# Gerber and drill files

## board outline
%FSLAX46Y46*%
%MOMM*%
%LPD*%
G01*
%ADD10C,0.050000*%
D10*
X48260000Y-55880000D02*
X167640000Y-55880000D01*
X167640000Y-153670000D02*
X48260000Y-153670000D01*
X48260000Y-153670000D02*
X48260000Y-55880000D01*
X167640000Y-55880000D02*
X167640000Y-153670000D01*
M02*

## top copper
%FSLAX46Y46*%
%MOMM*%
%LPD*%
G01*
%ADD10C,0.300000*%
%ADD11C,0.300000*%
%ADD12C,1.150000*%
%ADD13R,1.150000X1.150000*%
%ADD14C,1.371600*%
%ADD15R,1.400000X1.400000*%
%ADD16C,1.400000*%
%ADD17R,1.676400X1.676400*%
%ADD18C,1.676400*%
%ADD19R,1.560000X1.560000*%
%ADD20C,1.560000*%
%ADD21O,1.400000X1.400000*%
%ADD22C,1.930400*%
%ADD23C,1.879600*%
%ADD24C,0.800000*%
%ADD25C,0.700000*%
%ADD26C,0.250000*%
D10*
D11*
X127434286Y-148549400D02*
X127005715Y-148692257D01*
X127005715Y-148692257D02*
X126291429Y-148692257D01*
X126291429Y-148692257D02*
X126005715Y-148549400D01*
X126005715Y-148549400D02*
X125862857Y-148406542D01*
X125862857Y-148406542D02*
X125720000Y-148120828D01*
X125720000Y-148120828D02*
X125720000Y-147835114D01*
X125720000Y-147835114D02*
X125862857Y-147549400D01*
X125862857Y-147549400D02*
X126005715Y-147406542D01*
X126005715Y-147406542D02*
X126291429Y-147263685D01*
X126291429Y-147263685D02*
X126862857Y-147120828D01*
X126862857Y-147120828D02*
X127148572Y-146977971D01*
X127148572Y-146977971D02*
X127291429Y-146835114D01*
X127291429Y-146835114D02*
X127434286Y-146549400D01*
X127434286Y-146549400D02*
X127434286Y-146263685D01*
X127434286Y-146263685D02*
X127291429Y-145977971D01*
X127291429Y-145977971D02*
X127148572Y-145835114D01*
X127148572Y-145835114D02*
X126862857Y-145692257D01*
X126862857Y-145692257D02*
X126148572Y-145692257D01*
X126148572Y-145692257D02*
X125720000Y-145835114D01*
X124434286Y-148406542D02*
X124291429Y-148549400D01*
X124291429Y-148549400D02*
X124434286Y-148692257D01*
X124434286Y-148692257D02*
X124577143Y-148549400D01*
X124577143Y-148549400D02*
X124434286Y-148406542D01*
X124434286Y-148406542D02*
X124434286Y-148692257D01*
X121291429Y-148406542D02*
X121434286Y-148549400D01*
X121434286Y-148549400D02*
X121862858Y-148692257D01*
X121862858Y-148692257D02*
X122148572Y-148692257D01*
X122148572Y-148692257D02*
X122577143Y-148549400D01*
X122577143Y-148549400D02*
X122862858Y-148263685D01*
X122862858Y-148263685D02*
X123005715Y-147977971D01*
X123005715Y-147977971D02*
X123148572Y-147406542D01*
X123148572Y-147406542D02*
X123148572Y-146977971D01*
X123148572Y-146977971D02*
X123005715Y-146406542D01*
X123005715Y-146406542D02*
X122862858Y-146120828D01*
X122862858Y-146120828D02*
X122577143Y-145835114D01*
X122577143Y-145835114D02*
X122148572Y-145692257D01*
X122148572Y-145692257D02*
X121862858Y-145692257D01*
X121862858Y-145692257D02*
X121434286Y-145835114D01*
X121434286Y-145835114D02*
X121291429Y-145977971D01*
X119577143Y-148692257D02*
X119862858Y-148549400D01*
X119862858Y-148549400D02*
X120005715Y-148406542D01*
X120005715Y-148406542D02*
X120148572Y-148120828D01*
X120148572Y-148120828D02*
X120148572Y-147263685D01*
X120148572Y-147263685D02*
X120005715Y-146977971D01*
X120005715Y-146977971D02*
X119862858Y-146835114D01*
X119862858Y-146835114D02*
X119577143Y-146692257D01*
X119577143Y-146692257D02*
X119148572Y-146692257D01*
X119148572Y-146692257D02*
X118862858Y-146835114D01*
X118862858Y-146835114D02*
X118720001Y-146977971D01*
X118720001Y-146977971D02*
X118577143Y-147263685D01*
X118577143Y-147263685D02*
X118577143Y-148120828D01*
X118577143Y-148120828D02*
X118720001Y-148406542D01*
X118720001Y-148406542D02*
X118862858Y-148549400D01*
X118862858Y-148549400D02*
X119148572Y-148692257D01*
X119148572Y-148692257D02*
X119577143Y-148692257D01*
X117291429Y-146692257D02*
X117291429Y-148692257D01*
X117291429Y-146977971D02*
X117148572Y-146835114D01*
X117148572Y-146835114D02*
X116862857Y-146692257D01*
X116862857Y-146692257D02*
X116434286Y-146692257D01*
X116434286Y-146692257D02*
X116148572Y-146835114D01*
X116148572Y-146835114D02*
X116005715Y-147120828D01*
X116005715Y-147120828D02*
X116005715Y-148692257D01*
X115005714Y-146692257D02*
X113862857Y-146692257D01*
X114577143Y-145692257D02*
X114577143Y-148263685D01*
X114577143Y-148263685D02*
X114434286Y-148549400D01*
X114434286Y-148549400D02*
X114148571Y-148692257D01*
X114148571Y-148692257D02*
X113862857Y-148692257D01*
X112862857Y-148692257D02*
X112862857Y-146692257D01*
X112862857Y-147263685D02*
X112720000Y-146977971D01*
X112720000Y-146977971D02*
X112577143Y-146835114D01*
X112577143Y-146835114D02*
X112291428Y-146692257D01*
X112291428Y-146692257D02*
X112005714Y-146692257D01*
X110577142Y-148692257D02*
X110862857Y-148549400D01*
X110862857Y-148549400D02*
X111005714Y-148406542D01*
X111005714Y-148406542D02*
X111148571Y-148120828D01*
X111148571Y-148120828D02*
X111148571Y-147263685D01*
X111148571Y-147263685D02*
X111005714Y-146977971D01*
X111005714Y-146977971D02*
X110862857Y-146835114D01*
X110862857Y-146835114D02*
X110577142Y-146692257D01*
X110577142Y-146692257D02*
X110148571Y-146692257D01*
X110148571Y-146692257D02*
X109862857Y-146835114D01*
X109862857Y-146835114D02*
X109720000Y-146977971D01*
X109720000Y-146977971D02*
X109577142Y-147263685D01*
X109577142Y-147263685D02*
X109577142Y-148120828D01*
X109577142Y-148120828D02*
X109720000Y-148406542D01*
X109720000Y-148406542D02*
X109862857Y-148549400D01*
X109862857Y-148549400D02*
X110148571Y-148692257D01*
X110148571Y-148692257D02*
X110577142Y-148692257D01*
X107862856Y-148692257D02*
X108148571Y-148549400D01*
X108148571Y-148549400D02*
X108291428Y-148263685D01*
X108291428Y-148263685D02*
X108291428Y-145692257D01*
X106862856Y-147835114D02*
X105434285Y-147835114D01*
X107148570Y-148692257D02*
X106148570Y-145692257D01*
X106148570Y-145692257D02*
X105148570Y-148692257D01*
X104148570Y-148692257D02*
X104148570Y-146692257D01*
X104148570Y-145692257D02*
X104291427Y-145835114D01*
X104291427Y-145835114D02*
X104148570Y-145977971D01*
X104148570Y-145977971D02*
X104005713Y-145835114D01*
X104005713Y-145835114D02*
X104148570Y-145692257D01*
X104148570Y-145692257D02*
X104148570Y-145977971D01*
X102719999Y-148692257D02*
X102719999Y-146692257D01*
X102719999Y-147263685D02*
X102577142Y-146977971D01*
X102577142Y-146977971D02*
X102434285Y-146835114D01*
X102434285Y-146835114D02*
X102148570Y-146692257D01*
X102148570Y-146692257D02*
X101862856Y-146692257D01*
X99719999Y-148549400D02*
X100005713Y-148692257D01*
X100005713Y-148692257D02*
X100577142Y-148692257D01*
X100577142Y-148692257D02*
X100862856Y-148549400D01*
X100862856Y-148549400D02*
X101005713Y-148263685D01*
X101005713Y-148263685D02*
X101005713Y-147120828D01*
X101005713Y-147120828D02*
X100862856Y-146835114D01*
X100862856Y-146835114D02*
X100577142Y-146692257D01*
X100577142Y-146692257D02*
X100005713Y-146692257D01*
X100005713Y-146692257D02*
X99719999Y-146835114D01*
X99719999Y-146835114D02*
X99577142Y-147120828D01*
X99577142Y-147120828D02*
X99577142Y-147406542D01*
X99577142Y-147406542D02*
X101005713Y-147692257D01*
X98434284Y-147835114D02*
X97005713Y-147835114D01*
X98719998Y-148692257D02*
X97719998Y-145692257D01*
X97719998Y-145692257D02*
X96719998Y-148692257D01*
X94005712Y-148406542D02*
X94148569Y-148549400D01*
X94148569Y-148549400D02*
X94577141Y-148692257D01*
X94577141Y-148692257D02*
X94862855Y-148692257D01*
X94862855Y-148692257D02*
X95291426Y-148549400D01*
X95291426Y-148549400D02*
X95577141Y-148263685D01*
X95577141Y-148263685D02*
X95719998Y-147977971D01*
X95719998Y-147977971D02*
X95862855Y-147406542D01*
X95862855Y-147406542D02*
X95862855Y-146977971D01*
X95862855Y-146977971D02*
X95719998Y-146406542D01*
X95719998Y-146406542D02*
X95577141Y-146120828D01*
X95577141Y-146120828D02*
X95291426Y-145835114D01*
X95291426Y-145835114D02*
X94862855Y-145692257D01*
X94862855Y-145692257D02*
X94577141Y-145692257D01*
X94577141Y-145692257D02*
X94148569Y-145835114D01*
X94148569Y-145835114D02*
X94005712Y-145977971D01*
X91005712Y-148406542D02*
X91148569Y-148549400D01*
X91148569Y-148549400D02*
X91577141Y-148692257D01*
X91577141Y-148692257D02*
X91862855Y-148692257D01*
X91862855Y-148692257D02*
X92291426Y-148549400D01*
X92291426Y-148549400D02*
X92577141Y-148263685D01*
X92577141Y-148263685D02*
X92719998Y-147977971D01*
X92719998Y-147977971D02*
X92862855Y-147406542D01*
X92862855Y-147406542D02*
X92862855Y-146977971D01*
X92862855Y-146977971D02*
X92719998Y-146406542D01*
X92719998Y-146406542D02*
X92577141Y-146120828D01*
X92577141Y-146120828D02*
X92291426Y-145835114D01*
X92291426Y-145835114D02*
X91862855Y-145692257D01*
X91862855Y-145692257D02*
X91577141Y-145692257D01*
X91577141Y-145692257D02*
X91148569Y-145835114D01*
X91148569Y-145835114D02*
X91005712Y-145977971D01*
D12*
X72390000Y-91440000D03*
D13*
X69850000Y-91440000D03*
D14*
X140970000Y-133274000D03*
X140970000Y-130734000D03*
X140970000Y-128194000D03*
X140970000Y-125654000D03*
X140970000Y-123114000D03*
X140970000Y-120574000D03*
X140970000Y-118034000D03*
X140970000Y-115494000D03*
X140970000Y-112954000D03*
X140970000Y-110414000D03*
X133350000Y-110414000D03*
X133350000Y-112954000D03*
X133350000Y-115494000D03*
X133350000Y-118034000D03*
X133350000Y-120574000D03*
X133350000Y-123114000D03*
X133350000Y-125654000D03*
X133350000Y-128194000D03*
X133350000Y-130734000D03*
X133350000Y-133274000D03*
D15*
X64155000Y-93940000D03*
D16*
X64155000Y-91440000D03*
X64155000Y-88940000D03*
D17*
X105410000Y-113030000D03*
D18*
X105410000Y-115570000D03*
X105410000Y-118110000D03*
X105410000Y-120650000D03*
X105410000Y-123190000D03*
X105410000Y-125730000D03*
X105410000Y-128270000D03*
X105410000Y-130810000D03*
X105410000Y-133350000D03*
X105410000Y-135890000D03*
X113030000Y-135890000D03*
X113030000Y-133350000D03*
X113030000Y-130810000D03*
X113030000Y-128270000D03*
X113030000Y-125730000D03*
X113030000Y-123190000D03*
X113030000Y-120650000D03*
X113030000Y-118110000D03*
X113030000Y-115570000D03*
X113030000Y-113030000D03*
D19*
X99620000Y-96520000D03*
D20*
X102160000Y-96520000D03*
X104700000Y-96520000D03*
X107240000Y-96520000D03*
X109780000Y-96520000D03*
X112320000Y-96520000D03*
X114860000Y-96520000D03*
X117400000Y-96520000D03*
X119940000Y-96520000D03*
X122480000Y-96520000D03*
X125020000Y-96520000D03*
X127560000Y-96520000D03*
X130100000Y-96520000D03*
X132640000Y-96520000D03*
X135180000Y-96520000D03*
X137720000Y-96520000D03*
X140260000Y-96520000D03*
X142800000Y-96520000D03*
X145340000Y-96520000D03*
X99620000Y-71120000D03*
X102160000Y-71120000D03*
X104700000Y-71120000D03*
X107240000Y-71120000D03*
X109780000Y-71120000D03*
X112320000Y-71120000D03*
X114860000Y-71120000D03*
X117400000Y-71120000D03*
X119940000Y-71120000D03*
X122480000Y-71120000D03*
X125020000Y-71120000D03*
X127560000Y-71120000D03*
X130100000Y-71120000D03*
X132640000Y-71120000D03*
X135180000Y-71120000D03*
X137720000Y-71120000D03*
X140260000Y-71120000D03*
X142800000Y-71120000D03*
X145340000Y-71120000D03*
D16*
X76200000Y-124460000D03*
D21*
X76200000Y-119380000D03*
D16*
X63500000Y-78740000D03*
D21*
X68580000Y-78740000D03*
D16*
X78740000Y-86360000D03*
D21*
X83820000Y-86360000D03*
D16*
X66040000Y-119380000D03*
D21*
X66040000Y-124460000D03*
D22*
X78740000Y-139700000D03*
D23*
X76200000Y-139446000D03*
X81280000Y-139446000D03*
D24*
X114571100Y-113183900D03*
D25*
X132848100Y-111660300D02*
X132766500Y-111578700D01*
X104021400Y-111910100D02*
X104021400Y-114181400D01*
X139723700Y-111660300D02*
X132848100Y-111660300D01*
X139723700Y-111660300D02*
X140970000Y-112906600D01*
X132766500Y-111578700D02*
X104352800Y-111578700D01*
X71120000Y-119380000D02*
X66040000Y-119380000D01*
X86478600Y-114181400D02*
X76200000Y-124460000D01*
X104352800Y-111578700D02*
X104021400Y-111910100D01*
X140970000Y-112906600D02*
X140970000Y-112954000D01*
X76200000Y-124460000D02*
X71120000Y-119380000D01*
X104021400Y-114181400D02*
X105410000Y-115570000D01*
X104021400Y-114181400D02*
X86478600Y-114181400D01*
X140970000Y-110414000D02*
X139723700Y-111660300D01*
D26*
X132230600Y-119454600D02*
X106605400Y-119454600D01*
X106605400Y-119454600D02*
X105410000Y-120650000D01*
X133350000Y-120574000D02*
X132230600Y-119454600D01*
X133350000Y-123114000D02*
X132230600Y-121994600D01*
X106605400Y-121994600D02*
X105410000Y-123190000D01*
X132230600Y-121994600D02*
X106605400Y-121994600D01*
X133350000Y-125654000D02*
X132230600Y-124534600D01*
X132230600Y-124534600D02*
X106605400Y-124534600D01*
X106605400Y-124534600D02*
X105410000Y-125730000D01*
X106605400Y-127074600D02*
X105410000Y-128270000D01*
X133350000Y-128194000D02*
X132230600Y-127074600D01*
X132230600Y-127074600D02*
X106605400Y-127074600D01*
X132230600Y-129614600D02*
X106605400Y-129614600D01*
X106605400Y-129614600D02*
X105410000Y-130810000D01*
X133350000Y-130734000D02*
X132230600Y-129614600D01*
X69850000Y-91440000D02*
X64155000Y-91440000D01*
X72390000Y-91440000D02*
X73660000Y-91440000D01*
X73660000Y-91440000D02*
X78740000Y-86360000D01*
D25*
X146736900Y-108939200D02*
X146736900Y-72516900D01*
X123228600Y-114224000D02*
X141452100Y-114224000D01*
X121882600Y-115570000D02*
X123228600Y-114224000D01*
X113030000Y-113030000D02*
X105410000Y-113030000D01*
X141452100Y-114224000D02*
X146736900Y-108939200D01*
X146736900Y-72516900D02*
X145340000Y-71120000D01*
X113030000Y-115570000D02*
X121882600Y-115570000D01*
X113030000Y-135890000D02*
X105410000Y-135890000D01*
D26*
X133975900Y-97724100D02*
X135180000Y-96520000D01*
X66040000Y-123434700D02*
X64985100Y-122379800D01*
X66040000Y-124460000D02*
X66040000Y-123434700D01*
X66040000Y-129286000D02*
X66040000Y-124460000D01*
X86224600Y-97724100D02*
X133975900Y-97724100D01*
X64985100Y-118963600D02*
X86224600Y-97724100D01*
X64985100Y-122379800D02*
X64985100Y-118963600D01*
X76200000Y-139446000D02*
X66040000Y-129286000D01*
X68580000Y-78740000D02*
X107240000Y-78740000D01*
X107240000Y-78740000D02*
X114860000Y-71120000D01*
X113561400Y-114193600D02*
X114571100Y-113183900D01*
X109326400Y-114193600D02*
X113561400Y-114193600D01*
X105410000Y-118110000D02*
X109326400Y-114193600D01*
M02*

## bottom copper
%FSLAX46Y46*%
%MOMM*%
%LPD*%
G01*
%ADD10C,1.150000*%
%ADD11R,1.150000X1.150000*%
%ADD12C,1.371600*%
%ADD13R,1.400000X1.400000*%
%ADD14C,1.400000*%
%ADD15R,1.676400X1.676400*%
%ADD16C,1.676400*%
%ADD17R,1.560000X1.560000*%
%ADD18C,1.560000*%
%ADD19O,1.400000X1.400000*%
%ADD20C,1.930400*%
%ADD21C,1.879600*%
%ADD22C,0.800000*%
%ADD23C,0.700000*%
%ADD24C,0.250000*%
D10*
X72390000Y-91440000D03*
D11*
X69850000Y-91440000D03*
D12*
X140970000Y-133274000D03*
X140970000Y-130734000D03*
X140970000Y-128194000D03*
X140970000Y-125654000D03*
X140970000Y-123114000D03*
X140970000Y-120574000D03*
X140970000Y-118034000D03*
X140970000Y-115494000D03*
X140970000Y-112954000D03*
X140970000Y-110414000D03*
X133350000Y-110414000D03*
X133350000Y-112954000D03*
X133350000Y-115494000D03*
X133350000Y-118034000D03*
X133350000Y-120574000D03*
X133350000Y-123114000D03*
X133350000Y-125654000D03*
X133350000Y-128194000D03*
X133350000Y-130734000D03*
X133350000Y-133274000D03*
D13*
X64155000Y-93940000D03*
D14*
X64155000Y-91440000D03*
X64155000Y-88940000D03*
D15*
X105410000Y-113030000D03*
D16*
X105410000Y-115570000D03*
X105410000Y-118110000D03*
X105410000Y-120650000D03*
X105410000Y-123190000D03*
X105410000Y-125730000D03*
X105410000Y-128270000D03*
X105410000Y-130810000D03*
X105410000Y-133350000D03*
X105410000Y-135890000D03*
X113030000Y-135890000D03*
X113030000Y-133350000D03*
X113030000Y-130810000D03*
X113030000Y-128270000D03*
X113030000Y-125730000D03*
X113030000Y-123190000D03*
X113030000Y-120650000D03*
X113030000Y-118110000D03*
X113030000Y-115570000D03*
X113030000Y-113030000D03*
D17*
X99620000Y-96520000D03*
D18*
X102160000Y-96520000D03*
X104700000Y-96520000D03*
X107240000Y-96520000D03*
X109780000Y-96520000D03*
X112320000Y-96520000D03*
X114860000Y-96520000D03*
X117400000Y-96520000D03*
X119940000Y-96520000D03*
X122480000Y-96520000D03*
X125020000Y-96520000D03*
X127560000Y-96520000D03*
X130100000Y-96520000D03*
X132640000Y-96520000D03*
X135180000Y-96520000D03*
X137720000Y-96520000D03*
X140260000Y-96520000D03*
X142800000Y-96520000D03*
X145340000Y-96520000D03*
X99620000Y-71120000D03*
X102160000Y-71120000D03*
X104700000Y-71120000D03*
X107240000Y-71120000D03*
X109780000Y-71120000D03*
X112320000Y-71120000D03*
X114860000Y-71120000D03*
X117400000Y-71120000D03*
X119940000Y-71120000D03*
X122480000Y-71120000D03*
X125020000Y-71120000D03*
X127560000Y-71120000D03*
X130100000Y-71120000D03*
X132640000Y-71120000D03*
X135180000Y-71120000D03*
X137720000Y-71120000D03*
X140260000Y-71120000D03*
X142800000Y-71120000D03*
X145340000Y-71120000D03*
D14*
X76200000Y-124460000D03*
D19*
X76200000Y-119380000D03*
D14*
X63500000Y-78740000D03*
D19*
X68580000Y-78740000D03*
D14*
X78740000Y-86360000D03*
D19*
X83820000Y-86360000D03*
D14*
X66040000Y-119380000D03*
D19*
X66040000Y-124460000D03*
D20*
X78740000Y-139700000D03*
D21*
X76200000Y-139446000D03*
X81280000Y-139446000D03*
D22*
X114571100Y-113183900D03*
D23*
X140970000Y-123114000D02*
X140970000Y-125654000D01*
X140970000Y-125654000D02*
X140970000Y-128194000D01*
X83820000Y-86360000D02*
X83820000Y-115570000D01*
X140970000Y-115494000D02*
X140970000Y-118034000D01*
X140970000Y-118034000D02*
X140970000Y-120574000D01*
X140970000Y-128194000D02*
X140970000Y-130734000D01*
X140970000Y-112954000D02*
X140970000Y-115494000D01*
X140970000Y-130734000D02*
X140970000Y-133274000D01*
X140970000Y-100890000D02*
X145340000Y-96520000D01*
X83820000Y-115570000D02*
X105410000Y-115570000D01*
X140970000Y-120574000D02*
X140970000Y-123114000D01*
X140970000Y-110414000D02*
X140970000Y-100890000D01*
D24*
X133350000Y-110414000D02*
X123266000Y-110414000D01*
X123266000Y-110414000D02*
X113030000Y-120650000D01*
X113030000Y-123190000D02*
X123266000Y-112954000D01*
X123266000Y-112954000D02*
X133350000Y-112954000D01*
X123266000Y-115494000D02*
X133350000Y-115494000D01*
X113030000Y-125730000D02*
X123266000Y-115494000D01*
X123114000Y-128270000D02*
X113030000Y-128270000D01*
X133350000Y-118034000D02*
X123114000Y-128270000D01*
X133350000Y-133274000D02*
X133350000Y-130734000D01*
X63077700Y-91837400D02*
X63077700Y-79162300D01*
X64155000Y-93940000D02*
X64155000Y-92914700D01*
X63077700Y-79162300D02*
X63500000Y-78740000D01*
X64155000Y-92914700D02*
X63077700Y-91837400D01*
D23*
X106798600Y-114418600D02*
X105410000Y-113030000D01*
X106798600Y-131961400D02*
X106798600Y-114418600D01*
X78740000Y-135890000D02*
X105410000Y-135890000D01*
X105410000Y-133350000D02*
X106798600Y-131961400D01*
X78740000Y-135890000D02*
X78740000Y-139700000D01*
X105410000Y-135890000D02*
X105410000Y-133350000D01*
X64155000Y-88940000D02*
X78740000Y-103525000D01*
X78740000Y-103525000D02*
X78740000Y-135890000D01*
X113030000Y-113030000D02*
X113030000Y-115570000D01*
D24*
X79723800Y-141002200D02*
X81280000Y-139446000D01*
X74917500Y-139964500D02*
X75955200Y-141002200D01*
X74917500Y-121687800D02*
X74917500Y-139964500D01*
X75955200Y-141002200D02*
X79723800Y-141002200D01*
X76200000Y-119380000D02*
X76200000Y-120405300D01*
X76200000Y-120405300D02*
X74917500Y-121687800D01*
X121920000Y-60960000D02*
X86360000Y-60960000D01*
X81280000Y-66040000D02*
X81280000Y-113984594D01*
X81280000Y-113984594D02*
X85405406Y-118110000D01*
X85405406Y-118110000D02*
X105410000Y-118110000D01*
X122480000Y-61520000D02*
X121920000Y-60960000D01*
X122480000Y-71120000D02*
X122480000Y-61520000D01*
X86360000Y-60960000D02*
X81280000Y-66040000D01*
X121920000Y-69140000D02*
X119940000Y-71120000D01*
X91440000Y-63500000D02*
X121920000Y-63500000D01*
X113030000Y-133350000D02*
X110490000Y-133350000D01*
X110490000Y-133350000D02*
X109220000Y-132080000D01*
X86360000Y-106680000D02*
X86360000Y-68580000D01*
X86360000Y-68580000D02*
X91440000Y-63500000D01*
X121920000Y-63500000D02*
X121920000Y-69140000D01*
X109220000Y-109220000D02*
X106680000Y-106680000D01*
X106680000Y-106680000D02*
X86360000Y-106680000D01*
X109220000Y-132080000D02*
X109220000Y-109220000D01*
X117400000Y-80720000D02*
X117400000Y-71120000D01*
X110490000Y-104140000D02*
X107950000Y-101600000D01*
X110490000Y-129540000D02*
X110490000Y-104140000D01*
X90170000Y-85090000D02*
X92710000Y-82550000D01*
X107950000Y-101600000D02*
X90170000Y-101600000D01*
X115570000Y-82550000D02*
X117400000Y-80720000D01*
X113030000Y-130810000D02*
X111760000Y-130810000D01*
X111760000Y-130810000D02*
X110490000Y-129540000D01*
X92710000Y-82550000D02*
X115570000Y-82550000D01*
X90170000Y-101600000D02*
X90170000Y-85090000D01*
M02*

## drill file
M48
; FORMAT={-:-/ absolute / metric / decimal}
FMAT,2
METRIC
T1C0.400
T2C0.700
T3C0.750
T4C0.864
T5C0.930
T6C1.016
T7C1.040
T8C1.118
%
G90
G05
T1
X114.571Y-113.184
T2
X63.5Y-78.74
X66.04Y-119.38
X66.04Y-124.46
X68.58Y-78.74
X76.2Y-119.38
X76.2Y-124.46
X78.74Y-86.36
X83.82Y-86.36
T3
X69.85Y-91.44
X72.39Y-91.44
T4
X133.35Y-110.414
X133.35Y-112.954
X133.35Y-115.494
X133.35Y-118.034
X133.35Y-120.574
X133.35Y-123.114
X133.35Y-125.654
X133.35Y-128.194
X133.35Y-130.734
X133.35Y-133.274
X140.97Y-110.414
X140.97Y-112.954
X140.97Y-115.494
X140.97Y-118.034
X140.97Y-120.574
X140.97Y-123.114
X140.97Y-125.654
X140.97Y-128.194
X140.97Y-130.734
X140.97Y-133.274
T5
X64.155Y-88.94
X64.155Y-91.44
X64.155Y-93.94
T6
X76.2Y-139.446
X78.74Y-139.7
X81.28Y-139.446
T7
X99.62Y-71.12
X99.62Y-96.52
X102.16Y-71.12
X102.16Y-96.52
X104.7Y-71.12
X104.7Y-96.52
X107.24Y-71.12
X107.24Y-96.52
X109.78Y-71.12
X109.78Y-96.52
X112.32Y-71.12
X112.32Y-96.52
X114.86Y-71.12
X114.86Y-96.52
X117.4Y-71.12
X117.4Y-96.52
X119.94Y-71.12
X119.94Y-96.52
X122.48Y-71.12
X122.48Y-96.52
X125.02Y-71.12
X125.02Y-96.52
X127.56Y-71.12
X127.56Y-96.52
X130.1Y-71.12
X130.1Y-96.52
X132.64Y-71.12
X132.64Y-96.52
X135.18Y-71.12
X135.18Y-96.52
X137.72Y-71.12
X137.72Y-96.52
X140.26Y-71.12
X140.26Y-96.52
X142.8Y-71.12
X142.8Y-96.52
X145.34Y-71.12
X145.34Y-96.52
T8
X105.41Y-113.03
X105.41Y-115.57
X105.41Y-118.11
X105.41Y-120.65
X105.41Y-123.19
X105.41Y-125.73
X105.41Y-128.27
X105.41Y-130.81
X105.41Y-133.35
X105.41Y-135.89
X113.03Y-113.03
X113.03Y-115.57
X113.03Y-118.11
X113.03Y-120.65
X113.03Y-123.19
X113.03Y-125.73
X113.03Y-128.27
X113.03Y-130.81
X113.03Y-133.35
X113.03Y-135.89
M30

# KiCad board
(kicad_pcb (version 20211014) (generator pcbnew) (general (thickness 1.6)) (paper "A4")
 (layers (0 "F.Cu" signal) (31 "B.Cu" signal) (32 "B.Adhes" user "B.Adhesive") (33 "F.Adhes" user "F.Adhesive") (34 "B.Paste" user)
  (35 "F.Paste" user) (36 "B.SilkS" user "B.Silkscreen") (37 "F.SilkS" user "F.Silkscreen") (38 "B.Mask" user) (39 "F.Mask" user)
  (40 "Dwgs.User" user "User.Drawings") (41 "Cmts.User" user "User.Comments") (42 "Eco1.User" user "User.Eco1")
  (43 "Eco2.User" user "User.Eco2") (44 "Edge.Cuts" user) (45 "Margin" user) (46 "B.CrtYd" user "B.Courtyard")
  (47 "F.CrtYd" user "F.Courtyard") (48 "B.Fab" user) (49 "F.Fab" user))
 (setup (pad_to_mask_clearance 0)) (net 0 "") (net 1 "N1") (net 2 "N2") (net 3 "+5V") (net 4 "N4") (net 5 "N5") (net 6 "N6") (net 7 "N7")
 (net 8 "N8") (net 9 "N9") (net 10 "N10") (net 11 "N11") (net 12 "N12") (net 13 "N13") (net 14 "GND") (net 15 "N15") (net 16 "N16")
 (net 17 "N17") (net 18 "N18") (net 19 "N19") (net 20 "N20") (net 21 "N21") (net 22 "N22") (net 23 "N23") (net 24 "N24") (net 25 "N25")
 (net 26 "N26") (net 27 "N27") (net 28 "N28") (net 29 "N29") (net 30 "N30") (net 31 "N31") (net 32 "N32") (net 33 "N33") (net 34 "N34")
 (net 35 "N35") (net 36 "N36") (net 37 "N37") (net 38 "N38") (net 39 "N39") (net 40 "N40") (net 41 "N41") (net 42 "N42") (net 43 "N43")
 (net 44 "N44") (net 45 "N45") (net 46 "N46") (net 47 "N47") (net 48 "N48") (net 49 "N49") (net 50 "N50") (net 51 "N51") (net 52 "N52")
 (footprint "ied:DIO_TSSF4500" (layer "F.Cu") (at 71.12 91.44)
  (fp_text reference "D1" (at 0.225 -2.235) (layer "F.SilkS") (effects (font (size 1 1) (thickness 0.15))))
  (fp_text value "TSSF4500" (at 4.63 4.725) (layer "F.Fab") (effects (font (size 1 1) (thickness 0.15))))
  (pad "A" thru_hole circle locked (at 1.27 0) (size 1.15 1.15) (drill 0.75) (layers *.Cu *.Mask) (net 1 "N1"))
  (pad "C" thru_hole rect locked (at -1.27 0) (size 1.15 1.15) (drill 0.75) (layers *.Cu *.Mask) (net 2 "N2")))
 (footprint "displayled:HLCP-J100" (layer "F.Cu") (at 140.97 133.274 180)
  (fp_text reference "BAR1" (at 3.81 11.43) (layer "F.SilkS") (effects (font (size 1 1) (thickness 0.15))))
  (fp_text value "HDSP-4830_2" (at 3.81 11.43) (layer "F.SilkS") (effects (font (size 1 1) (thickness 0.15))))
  (pad "1" thru_hole circle locked (at 0 0 180) (size 1.3716 1.3716) (drill 0.8636) (layers *.Cu *.Mask) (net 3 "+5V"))
  (pad "2" thru_hole circle locked (at 0 2.54 180) (size 1.3716 1.3716) (drill 0.8636) (layers *.Cu *.Mask) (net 3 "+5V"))
  (pad "3" thru_hole circle locked (at 0 5.08 180) (size 1.3716 1.3716) (drill 0.8636) (layers *.Cu *.Mask) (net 3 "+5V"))
  (pad "4" thru_hole circle locked (at 0 7.62 180) (size 1.3716 1.3716) (drill 0.8636) (layers *.Cu *.Mask) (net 3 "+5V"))
  (pad "5" thru_hole circle locked (at 0 10.16 180) (size 1.3716 1.3716) (drill 0.8636) (layers *.Cu *.Mask) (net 3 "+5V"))
  (pad "6" thru_hole circle locked (at 0 12.7 180) (size 1.3716 1.3716) (drill 0.8636) (layers *.Cu *.Mask) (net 3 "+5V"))
  (pad "7" thru_hole circle locked (at 0 15.24 180) (size 1.3716 1.3716) (drill 0.8636) (layers *.Cu *.Mask) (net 3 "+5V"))
  (pad "8" thru_hole circle locked (at 0 17.78 180) (size 1.3716 1.3716) (drill 0.8636) (layers *.Cu *.Mask) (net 3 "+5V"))
  (pad "9" thru_hole circle locked (at 0 20.32 180) (size 1.3716 1.3716) (drill 0.8636) (layers *.Cu *.Mask) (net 3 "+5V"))
  (pad "10" thru_hole circle locked (at 0 22.86 180) (size 1.3716 1.3716) (drill 0.8636) (layers *.Cu *.Mask) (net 3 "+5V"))
  (pad "11" thru_hole circle locked (at 7.62 22.86 180) (size 1.3716 1.3716) (drill 0.8636) (layers *.Cu *.Mask) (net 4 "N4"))
  (pad "12" thru_hole circle locked (at 7.62 20.32 180) (size 1.3716 1.3716) (drill 0.8636) (layers *.Cu *.Mask) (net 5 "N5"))
  (pad "13" thru_hole circle locked (at 7.62 17.78 180) (size 1.3716 1.3716) (drill 0.8636) (layers *.Cu *.Mask) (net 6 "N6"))
  (pad "14" thru_hole circle locked (at 7.62 15.24 180) (size 1.3716 1.3716) (drill 0.8636) (layers *.Cu *.Mask) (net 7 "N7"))
  (pad "15" thru_hole circle locked (at 7.62 12.7 180) (size 1.3716 1.3716) (drill 0.8636) (layers *.Cu *.Mask) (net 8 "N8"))
  (pad "16" thru_hole circle locked (at 7.62 10.16 180) (size 1.3716 1.3716) (drill 0.8636) (layers *.Cu *.Mask) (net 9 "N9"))
  (pad "17" thru_hole circle locked (at 7.62 7.62 180) (size 1.3716 1.3716) (drill 0.8636) (layers *.Cu *.Mask) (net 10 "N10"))
  (pad "18" thru_hole circle locked (at 7.62 5.08 180) (size 1.3716 1.3716) (drill 0.8636) (layers *.Cu *.Mask) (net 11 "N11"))
  (pad "19" thru_hole circle locked (at 7.62 2.54 180) (size 1.3716 1.3716) (drill 0.8636) (layers *.Cu *.Mask) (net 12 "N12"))
  (pad "20" thru_hole circle locked (at 7.62 0 180) (size 1.3716 1.3716) (drill 0.8636) (layers *.Cu *.Mask) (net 12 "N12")))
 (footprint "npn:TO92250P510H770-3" (layer "F.Cu") (at 63.5 91.44 90)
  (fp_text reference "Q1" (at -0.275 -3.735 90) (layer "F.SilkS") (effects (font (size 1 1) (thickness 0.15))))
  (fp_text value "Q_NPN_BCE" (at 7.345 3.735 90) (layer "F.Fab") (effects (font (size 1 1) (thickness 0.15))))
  (pad "1" thru_hole rect locked (at -2.5 0.655 90) (size 1.4 1.4) (drill 0.93) (layers *.Cu *.Mask) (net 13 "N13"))
  (pad "2" thru_hole circle locked (at 0 0.655 90) (size 1.4 1.4) (drill 0.93) (layers *.Cu *.Mask) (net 2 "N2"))
  (pad "3" thru_hole circle locked (at 2.5 0.655 90) (size 1.4 1.4) (drill 0.93) (layers *.Cu *.Mask) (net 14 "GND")))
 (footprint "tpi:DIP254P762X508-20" (layer "F.Cu") (at 113.03 135.89)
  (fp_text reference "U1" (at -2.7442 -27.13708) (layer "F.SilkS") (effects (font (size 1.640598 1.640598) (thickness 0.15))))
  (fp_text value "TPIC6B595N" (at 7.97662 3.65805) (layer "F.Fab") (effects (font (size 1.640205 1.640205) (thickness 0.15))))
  (pad "1" thru_hole rect locked (at -7.62 -22.86) (size 1.6764 1.6764) (drill 1.1176) (layers *.Cu *.Mask) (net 14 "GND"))
  (pad "2" thru_hole circle locked (at -7.62 -20.32) (size 1.6764 1.6764) (drill 1.1176) (layers *.Cu *.Mask) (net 3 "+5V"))
  (pad "3" thru_hole circle locked (at -7.62 -17.78) (size 1.6764 1.6764) (drill 1.1176) (layers *.Cu *.Mask) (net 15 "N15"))
  (pad "4" thru_hole circle locked (at -7.62 -15.24) (size 1.6764 1.6764) (drill 1.1176) (layers *.Cu *.Mask) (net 8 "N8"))
  (pad "5" thru_hole circle locked (at -7.62 -12.7) (size 1.6764 1.6764) (drill 1.1176) (layers *.Cu *.Mask) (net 9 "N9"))
  (pad "6" thru_hole circle locked (at -7.62 -10.16) (size 1.6764 1.6764) (drill 1.1176) (layers *.Cu *.Mask) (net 10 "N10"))
  (pad "7" thru_hole circle locked (at -7.62 -7.62) (size 1.6764 1.6764) (drill 1.1176) (layers *.Cu *.Mask) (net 11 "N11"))
  (pad "8" thru_hole circle locked (at -7.62 -5.08) (size 1.6764 1.6764) (drill 1.1176) (layers *.Cu *.Mask) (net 12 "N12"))
  (pad "9" thru_hole circle locked (at -7.62 -2.54) (size 1.6764 1.6764) (drill 1.1176) (layers *.Cu *.Mask) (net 14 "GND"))
  (pad "10" thru_hole circle locked (at -7.62 0) (size 1.6764 1.6764) (drill 1.1176) (layers *.Cu *.Mask) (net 14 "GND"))
  (pad "11" thru_hole circle locked (at 0 0) (size 1.6764 1.6764) (drill 1.1176) (layers *.Cu *.Mask) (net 14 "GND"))
  (pad "12" thru_hole circle locked (at 0 -2.54) (size 1.6764 1.6764) (drill 1.1176) (layers *.Cu *.Mask) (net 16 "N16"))
  (pad "13" thru_hole circle locked (at 0 -5.08) (size 1.6764 1.6764) (drill 1.1176) (layers *.Cu *.Mask) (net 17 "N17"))
  (pad "14" thru_hole circle locked (at 0 -7.62) (size 1.6764 1.6764) (drill 1.1176) (layers *.Cu *.Mask) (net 7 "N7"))
  (pad "15" thru_hole circle locked (at 0 -10.16) (size 1.6764 1.6764) (drill 1.1176) (layers *.Cu *.Mask) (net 6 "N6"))
  (pad "16" thru_hole circle locked (at 0 -12.7) (size 1.6764 1.6764) (drill 1.1176) (layers *.Cu *.Mask) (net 5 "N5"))
  (pad "17" thru_hole circle locked (at 0 -15.24) (size 1.6764 1.6764) (drill 1.1176) (layers *.Cu *.Mask) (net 4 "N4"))
  (pad "18" thru_hole circle locked (at 0 -17.78) (size 1.6764 1.6764) (drill 1.1176) (layers *.Cu *.Mask) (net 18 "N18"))
  (pad "19" thru_hole circle locked (at 0 -20.32) (size 1.6764 1.6764) (drill 1.1176) (layers *.Cu *.Mask) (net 14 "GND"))
  (pad "20" thru_hole circle locked (at 0 -22.86) (size 1.6764 1.6764) (drill 1.1176) (layers *.Cu *.Mask) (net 14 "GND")))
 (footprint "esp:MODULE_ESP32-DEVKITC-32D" (layer "F.Cu") (at 119.38 83.82 90)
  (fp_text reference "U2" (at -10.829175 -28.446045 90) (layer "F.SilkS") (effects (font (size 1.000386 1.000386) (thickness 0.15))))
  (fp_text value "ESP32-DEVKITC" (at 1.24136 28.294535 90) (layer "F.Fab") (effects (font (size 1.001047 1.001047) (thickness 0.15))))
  (pad "1" thru_hole rect locked (at -12.7 -19.76 90) (size 1.56 1.56) (drill 1.04) (layers *.Cu *.Mask) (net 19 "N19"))
  (pad "2" thru_hole circle locked (at -12.7 -17.22 90) (size 1.56 1.56) (drill 1.04) (layers *.Cu *.Mask) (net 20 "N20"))
  (pad "3" thru_hole circle locked (at -12.7 -14.68 90) (size 1.56 1.56) (drill 1.04) (layers *.Cu *.Mask) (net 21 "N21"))
  (pad "4" thru_hole circle locked (at -12.7 -12.14 90) (size 1.56 1.56) (drill 1.04) (layers *.Cu *.Mask) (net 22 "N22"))
  (pad "5" thru_hole circle locked (at -12.7 -9.6 90) (size 1.56 1.56) (drill 1.04) (layers *.Cu *.Mask) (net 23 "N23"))
  (pad "6" thru_hole circle locked (at -12.7 -7.06 90) (size 1.56 1.56) (drill 1.04) (layers *.Cu *.Mask) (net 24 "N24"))
  (pad "7" thru_hole circle locked (at -12.7 -4.52 90) (size 1.56 1.56) (drill 1.04) (layers *.Cu *.Mask) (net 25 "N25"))
  (pad "8" thru_hole circle locked (at -12.7 -1.98 90) (size 1.56 1.56) (drill 1.04) (layers *.Cu *.Mask) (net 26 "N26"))
  (pad "9" thru_hole circle locked (at -12.7 0.56 90) (size 1.56 1.56) (drill 1.04) (layers *.Cu *.Mask) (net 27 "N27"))
  (pad "10" thru_hole circle locked (at -12.7 3.1 90) (size 1.56 1.56) (drill 1.04) (layers *.Cu *.Mask) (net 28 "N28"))
  (pad "11" thru_hole circle locked (at -12.7 5.64 90) (size 1.56 1.56) (drill 1.04) (layers *.Cu *.Mask) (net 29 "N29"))
  (pad "12" thru_hole circle locked (at -12.7 8.18 90) (size 1.56 1.56) (drill 1.04) (layers *.Cu *.Mask) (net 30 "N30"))
  (pad "13" thru_hole circle locked (at -12.7 10.72 90) (size 1.56 1.56) (drill 1.04) (layers *.Cu *.Mask) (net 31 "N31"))
  (pad "14" thru_hole circle locked (at -12.7 13.26 90) (size 1.56 1.56) (drill 1.04) (layers *.Cu *.Mask) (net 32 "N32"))
  (pad "15" thru_hole circle locked (at -12.7 15.8 90) (size 1.56 1.56) (drill 1.04) (layers *.Cu *.Mask) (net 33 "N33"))
  (pad "16" thru_hole circle locked (at -12.7 18.34 90) (size 1.56 1.56) (drill 1.04) (layers *.Cu *.Mask) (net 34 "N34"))
  (pad "17" thru_hole circle locked (at -12.7 20.88 90) (size 1.56 1.56) (drill 1.04) (layers *.Cu *.Mask) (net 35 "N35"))
  (pad "18" thru_hole circle locked (at -12.7 23.42 90) (size 1.56 1.56) (drill 1.04) (layers *.Cu *.Mask) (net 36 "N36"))
  (pad "19" thru_hole circle locked (at -12.7 25.96 90) (size 1.56 1.56) (drill 1.04) (layers *.Cu *.Mask) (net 3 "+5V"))
  (pad "20" thru_hole circle locked (at 12.7 -19.76 90) (size 1.56 1.56) (drill 1.04) (layers *.Cu *.Mask) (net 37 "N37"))
  (pad "21" thru_hole circle locked (at 12.7 -17.22 90) (size 1.56 1.56) (drill 1.04) (layers *.Cu *.Mask) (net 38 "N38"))
  (pad "22" thru_hole circle locked (at 12.7 -14.68 90) (size 1.56 1.56) (drill 1.04) (layers *.Cu *.Mask) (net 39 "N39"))
  (pad "23" thru_hole circle locked (at 12.7 -12.14 90) (size 1.56 1.56) (drill 1.04) (layers *.Cu *.Mask) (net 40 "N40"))
  (pad "24" thru_hole circle locked (at 12.7 -9.6 90) (size 1.56 1.56) (drill 1.04) (layers *.Cu *.Mask) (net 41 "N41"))
  (pad "25" thru_hole circle locked (at 12.7 -7.06 90) (size 1.56 1.56) (drill 1.04) (layers *.Cu *.Mask) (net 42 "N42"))
  (pad "26" thru_hole circle locked (at 12.7 -4.52 90) (size 1.56 1.56) (drill 1.04) (layers *.Cu *.Mask) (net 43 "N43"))
  (pad "27" thru_hole circle locked (at 12.7 -1.98 90) (size 1.56 1.56) (drill 1.04) (layers *.Cu *.Mask) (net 17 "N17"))
  (pad "28" thru_hole circle locked (at 12.7 0.56 90) (size 1.56 1.56) (drill 1.04) (layers *.Cu *.Mask) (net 16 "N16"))
  (pad "29" thru_hole circle locked (at 12.7 3.1 90) (size 1.56 1.56) (drill 1.04) (layers *.Cu *.Mask) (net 15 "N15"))
  (pad "30" thru_hole circle locked (at 12.7 5.64 90) (size 1.56 1.56) (drill 1.04) (layers *.Cu *.Mask) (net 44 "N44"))
  (pad "31" thru_hole circle locked (at 12.7 8.18 90) (size 1.56 1.56) (drill 1.04) (layers *.Cu *.Mask) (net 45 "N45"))
  (pad "32" thru_hole circle locked (at 12.7 10.72 90) (size 1.56 1.56) (drill 1.04) (layers *.Cu *.Mask) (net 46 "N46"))
  (pad "33" thru_hole circle locked (at 12.7 13.26 90) (size 1.56 1.56) (drill 1.04) (layers *.Cu *.Mask) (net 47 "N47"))
  (pad "34" thru_hole circle locked (at 12.7 15.8 90) (size 1.56 1.56) (drill 1.04) (layers *.Cu *.Mask) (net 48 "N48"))
  (pad "35" thru_hole circle locked (at 12.7 18.34 90) (size 1.56 1.56) (drill 1.04) (layers *.Cu *.Mask) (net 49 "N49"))
  (pad "36" thru_hole circle locked (at 12.7 20.88 90) (size 1.56 1.56) (drill 1.04) (layers *.Cu *.Mask) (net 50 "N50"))
  (pad "37" thru_hole circle locked (at 12.7 23.42 90) (size 1.56 1.56) (drill 1.04) (layers *.Cu *.Mask) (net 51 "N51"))
  (pad "38" thru_hole circle locked (at 12.7 25.96 90) (size 1.56 1.56) (drill 1.04) (layers *.Cu *.Mask) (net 14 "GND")))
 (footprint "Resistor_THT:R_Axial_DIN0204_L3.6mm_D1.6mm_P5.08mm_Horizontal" (layer "F.Cu") (at 76.2 124.46 90)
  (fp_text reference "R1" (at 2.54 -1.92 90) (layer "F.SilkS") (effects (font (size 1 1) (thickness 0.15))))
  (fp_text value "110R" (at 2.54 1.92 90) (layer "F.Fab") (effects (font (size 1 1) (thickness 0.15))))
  (pad "1" thru_hole circle (at 0 0 90) (size 1.4 1.4) (drill 0.7) (layers *.Cu *.Mask) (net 3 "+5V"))
  (pad "2" thru_hole oval (at 5.08 0 90) (size 1.4 1.4) (drill 0.7) (layers *.Cu *.Mask) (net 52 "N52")))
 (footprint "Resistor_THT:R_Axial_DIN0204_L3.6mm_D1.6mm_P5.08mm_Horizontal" (layer "F.Cu") (at 63.5 78.74)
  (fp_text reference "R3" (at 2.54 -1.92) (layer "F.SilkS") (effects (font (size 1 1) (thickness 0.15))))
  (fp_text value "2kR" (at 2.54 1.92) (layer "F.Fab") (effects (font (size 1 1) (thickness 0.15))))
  (pad "1" thru_hole circle (at 0 0) (size 1.4 1.4) (drill 0.7) (layers *.Cu *.Mask) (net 13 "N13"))
  (pad "2" thru_hole oval (at 5.08 0) (size 1.4 1.4) (drill 0.7) (layers *.Cu *.Mask) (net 43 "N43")))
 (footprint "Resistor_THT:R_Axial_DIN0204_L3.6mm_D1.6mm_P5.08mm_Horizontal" (layer "F.Cu") (at 78.74 86.36)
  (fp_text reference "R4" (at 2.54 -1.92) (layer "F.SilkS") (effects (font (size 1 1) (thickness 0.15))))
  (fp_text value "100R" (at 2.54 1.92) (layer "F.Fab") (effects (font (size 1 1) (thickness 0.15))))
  (pad "1" thru_hole circle (at 0 0) (size 1.4 1.4) (drill 0.7) (layers *.Cu *.Mask) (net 1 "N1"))
  (pad "2" thru_hole oval (at 5.08 0) (size 1.4 1.4) (drill 0.7) (layers *.Cu *.Mask) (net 3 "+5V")))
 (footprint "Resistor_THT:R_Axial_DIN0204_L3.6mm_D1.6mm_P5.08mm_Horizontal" (layer "F.Cu") (at 66.04 119.38 -90)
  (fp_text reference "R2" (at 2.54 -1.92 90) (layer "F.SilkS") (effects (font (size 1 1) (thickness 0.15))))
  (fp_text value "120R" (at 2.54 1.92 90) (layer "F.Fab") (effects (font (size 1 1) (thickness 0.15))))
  (pad "1" thru_hole circle (at 0 0 270) (size 1.4 1.4) (drill 0.7) (layers *.Cu *.Mask) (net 3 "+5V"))
  (pad "2" thru_hole oval (at 5.08 0 270) (size 1.4 1.4) (drill 0.7) (layers *.Cu *.Mask) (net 33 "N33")))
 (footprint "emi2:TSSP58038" (layer "F.Cu") (at 78.74 139.7 -90)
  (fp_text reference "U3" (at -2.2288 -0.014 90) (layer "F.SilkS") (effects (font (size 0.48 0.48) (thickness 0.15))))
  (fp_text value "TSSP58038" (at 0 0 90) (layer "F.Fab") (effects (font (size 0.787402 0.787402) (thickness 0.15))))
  (pad "GND" thru_hole circle locked (at 0 0 270) (size 1.9304 1.9304) (drill 1.016) (layers *.Cu *.Mask) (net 14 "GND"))
  (pad "OUT" thru_hole circle locked (at -0.254 2.54 270) (size 1.8796 1.8796) (drill 1.016) (layers *.Cu *.Mask) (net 33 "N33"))
  (pad "VS" thru_hole circle locked (at -0.254 -2.54 270) (size 1.8796 1.8796) (drill 1.016) (layers *.Cu *.Mask) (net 52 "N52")))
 (gr_line (start 48.26 55.88) (end 167.64 55.88) (layer "Edge.Cuts") (width 0.05))
 (gr_line (start 167.64 153.67) (end 48.26 153.67) (layer "Edge.Cuts") (width 0.05))
 (gr_line (start 48.26 153.67) (end 48.26 55.88) (layer "Edge.Cuts") (width 0.05))
 (gr_line (start 167.64 55.88) (end 167.64 153.67) (layer "Edge.Cuts") (width 0.05))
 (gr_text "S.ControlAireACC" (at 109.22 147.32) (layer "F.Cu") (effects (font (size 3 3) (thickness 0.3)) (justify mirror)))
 (segment (start 132.8481 111.6603) (end 132.7665 111.5787) (width 0.7) (layer "F.Cu") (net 3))
 (segment (start 104.0214 111.9101) (end 104.0214 114.1814) (width 0.7) (layer "F.Cu") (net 3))
 (segment (start 139.7237 111.6603) (end 132.8481 111.6603) (width 0.7) (layer "F.Cu") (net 3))
 (segment (start 139.7237 111.6603) (end 140.97 112.9066) (width 0.7) (layer "F.Cu") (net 3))
 (segment (start 132.7665 111.5787) (end 104.3528 111.5787) (width 0.7) (layer "F.Cu") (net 3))
 (segment (start 71.12 119.38) (end 66.04 119.38) (width 0.7) (layer "F.Cu") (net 3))
 (segment (start 86.4786 114.1814) (end 76.2 124.46) (width 0.7) (layer "F.Cu") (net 3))
 (segment (start 104.3528 111.5787) (end 104.0214 111.9101) (width 0.7) (layer "F.Cu") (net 3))
 (segment (start 140.97 112.9066) (end 140.97 112.954) (width 0.7) (layer "F.Cu") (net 3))
 (segment (start 76.2 124.46) (end 71.12 119.38) (width 0.7) (layer "F.Cu") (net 3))
 (segment (start 104.0214 114.1814) (end 105.41 115.57) (width 0.7) (layer "F.Cu") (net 3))
 (segment (start 104.0214 114.1814) (end 86.4786 114.1814) (width 0.7) (layer "F.Cu") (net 3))
 (segment (start 140.97 110.414) (end 139.7237 111.6603) (width 0.7) (layer "F.Cu") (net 3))
 (segment (start 140.97 123.114) (end 140.97 125.654) (width 0.7) (layer "B.Cu") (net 3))
 (segment (start 140.97 125.654) (end 140.97 128.194) (width 0.7) (layer "B.Cu") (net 3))
 (segment (start 83.82 86.36) (end 83.82 115.57) (width 0.7) (layer "B.Cu") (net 3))
 (segment (start 140.97 115.494) (end 140.97 118.034) (width 0.7) (layer "B.Cu") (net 3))
 (segment (start 140.97 118.034) (end 140.97 120.574) (width 0.7) (layer "B.Cu") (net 3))
 (segment (start 140.97 128.194) (end 140.97 130.734) (width 0.7) (layer "B.Cu") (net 3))
 (segment (start 140.97 112.954) (end 140.97 115.494) (width 0.7) (layer "B.Cu") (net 3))
 (segment (start 140.97 130.734) (end 140.97 133.274) (width 0.7) (layer "B.Cu") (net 3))
 (segment (start 140.97 100.89) (end 145.34 96.52) (width 0.7) (layer "B.Cu") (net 3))
 (segment (start 83.82 115.57) (end 105.41 115.57) (width 0.7) (layer "B.Cu") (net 3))
 (segment (start 140.97 120.574) (end 140.97 123.114) (width 0.7) (layer "B.Cu") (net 3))
 (segment (start 140.97 110.414) (end 140.97 100.89) (width 0.7) (layer "B.Cu") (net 3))
 (segment (start 133.35 110.414) (end 123.266 110.414) (width 0.25) (layer "B.Cu") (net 4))
 (segment (start 123.266 110.414) (end 113.03 120.65) (width 0.25) (layer "B.Cu") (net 4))
 (segment (start 113.03 123.19) (end 123.266 112.954) (width 0.25) (layer "B.Cu") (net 5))
 (segment (start 123.266 112.954) (end 133.35 112.954) (width 0.25) (layer "B.Cu") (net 5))
 (segment (start 123.266 115.494) (end 133.35 115.494) (width 0.25) (layer "B.Cu") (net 6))
 (segment (start 113.03 125.73) (end 123.266 115.494) (width 0.25) (layer "B.Cu") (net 6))
 (segment (start 123.114 128.27) (end 113.03 128.27) (width 0.25) (layer "B.Cu") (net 7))
 (segment (start 133.35 118.034) (end 123.114 128.27) (width 0.25) (layer "B.Cu") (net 7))
 (segment (start 132.2306 119.4546) (end 106.6054 119.4546) (width 0.25) (layer "F.Cu") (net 8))
 (segment (start 106.6054 119.4546) (end 105.41 120.65) (width 0.25) (layer "F.Cu") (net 8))
 (segment (start 133.35 120.574) (end 132.2306 119.4546) (width 0.25) (layer "F.Cu") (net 8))
 (segment (start 133.35 123.114) (end 132.2306 121.9946) (width 0.25) (layer "F.Cu") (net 9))
 (segment (start 106.6054 121.9946) (end 105.41 123.19) (width 0.25) (layer "F.Cu") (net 9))
 (segment (start 132.2306 121.9946) (end 106.6054 121.9946) (width 0.25) (layer "F.Cu") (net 9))
 (segment (start 133.35 125.654) (end 132.2306 124.5346) (width 0.25) (layer "F.Cu") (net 10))
 (segment (start 132.2306 124.5346) (end 106.6054 124.5346) (width 0.25) (layer "F.Cu") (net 10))
 (segment (start 106.6054 124.5346) (end 105.41 125.73) (width 0.25) (layer "F.Cu") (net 10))
 (segment (start 106.6054 127.0746) (end 105.41 128.27) (width 0.25) (layer "F.Cu") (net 11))
 (segment (start 133.35 128.194) (end 132.2306 127.0746) (width 0.25) (layer "F.Cu") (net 11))
 (segment (start 132.2306 127.0746) (end 106.6054 127.0746) (width 0.25) (layer "F.Cu") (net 11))
 (segment (start 132.2306 129.6146) (end 106.6054 129.6146) (width 0.25) (layer "F.Cu") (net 12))
 (segment (start 106.6054 129.6146) (end 105.41 130.81) (width 0.25) (layer "F.Cu") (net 12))
 (segment (start 133.35 130.734) (end 132.2306 129.6146) (width 0.25) (layer "F.Cu") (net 12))
 (segment (start 133.35 133.274) (end 133.35 130.734) (width 0.25) (layer "B.Cu") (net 12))
 (segment (start 69.85 91.44) (end 64.155 91.44) (width 0.25) (layer "F.Cu") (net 2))
 (segment (start 72.39 91.44) (end 73.66 91.44) (width 0.25) (layer "F.Cu") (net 1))
 (segment (start 73.66 91.44) (end 78.74 86.36) (width 0.25) (layer "F.Cu") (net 1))
 (segment (start 63.0777 91.8374) (end 63.0777 79.1623) (width 0.25) (layer "B.Cu") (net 13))
 (segment (start 64.155 93.94) (end 64.155 92.9147) (width 0.25) (layer "B.Cu") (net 13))
 (segment (start 63.0777 79.1623) (end 63.5 78.74) (width 0.25) (layer "B.Cu") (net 13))
 (segment (start 64.155 92.9147) (end 63.0777 91.8374) (width 0.25) (layer "B.Cu") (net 13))
 (segment (start 146.7369 108.9392) (end 146.7369 72.5169) (width 0.7) (layer "F.Cu") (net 14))
 (segment (start 123.2286 114.224) (end 141.4521 114.224) (width 0.7) (layer "F.Cu") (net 14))
 (segment (start 121.8826 115.57) (end 123.2286 114.224) (width 0.7) (layer "F.Cu") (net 14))
 (segment (start 113.03 113.03) (end 105.41 113.03) (width 0.7) (layer "F.Cu") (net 14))
 (segment (start 141.4521 114.224) (end 146.7369 108.9392) (width 0.7) (layer "F.Cu") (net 14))
 (segment (start 146.7369 72.5169) (end 145.34 71.12) (width 0.7) (layer "F.Cu") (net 14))
 (segment (start 113.03 115.57) (end 121.8826 115.57) (width 0.7) (layer "F.Cu") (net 14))
 (segment (start 113.03 135.89) (end 105.41 135.89) (width 0.7) (layer "F.Cu") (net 14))
 (segment (start 106.7986 114.4186) (end 105.41 113.03) (width 0.7) (layer "B.Cu") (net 14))
 (segment (start 106.7986 131.9614) (end 106.7986 114.4186) (width 0.7) (layer "B.Cu") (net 14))
 (segment (start 78.74 135.89) (end 105.41 135.89) (width 0.7) (layer "B.Cu") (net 14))
 (segment (start 105.41 133.35) (end 106.7986 131.9614) (width 0.7) (layer "B.Cu") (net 14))
 (segment (start 78.74 135.89) (end 78.74 139.7) (width 0.7) (layer "B.Cu") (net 14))
 (segment (start 105.41 135.89) (end 105.41 133.35) (width 0.7) (layer "B.Cu") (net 14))
 (segment (start 64.155 88.94) (end 78.74 103.525) (width 0.7) (layer "B.Cu") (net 14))
 (segment (start 78.74 103.525) (end 78.74 135.89) (width 0.7) (layer "B.Cu") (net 14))
 (segment (start 113.03 113.03) (end 113.03 115.57) (width 0.7) (layer "B.Cu") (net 14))
 (segment (start 79.7238 141.0022) (end 81.28 139.446) (width 0.25) (layer "B.Cu") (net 52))
 (segment (start 74.9175 139.9645) (end 75.9552 141.0022) (width 0.25) (layer "B.Cu") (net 52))
 (segment (start 74.9175 121.6878) (end 74.9175 139.9645) (width 0.25) (layer "B.Cu") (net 52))
 (segment (start 75.9552 141.0022) (end 79.7238 141.0022) (width 0.25) (layer "B.Cu") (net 52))
 (segment (start 76.2 119.38) (end 76.2 120.4053) (width 0.25) (layer "B.Cu") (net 52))
 (segment (start 76.2 120.4053) (end 74.9175 121.6878) (width 0.25) (layer "B.Cu") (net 52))
 (segment (start 133.9759 97.7241) (end 135.18 96.52) (width 0.25) (layer "F.Cu") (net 33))
 (segment (start 66.04 123.4347) (end 64.9851 122.3798) (width 0.25) (layer "F.Cu") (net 33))
 (segment (start 66.04 124.46) (end 66.04 123.4347) (width 0.25) (layer "F.Cu") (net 33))
 (segment (start 66.04 129.286) (end 66.04 124.46) (width 0.25) (layer "F.Cu") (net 33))
 (segment (start 86.2246 97.7241) (end 133.9759 97.7241) (width 0.25) (layer "F.Cu") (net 33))
 (segment (start 64.9851 118.9636) (end 86.2246 97.7241) (width 0.25) (layer "F.Cu") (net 33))
 (segment (start 64.9851 122.3798) (end 64.9851 118.9636) (width 0.25) (layer "F.Cu") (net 33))
 (segment (start 76.2 139.446) (end 66.04 129.286) (width 0.25) (layer "F.Cu") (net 33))
 (segment (start 68.58 78.74) (end 107.24 78.74) (width 0.25) (layer "F.Cu") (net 43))
 (segment (start 107.24 78.74) (end 114.86 71.12) (width 0.25) (layer "F.Cu") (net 43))
 (segment (start 113.5614 114.1936) (end 114.5711 113.1839) (width 0.25) (layer "F.Cu") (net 15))
 (segment (start 109.3264 114.1936) (end 113.5614 114.1936) (width 0.25) (layer "F.Cu") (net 15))
 (segment (start 105.41 118.11) (end 109.3264 114.1936) (width 0.25) (layer "F.Cu") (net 15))
 (via (at 114.5711 113.1839) (size 0.8) (drill 0.4) (layers "F.Cu" "B.Cu") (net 15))
 (segment (start 121.92 60.96) (end 86.36 60.96) (width 0.25) (layer "B.Cu") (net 15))
 (segment (start 81.28 66.04) (end 81.28 113.984594) (width 0.25) (layer "B.Cu") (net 15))
 (segment (start 81.28 113.984594) (end 85.405406 118.11) (width 0.25) (layer "B.Cu") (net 15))
 (segment (start 85.405406 118.11) (end 105.41 118.11) (width 0.25) (layer "B.Cu") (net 15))
 (segment (start 122.48 61.52) (end 121.92 60.96) (width 0.25) (layer "B.Cu") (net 15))
 (segment (start 122.48 71.12) (end 122.48 61.52) (width 0.25) (layer "B.Cu") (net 15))
 (segment (start 86.36 60.96) (end 81.28 66.04) (width 0.25) (layer "B.Cu") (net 15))
 (segment (start 121.92 69.14) (end 119.94 71.12) (width 0.25) (layer "B.Cu") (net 16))
 (segment (start 91.44 63.5) (end 121.92 63.5) (width 0.25) (layer "B.Cu") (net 16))
 (segment (start 113.03 133.35) (end 110.49 133.35) (width 0.25) (layer "B.Cu") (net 16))
 (segment (start 110.49 133.35) (end 109.22 132.08) (width 0.25) (layer "B.Cu") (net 16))
 (segment (start 86.36 106.68) (end 86.36 68.58) (width 0.25) (layer "B.Cu") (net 16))
 (segment (start 86.36 68.58) (end 91.44 63.5) (width 0.25) (layer "B.Cu") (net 16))
 (segment (start 121.92 63.5) (end 121.92 69.14) (width 0.25) (layer "B.Cu") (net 16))
 (segment (start 109.22 109.22) (end 106.68 106.68) (width 0.25) (layer "B.Cu") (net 16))
 (segment (start 106.68 106.68) (end 86.36 106.68) (width 0.25) (layer "B.Cu") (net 16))
 (segment (start 109.22 132.08) (end 109.22 109.22) (width 0.25) (layer "B.Cu") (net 16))
 (segment (start 117.4 80.72) (end 117.4 71.12) (width 0.25) (layer "B.Cu") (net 17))
 (segment (start 110.49 104.14) (end 107.95 101.6) (width 0.25) (layer "B.Cu") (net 17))
 (segment (start 110.49 129.54) (end 110.49 104.14) (width 0.25) (layer "B.Cu") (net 17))
 (segment (start 90.17 85.09) (end 92.71 82.55) (width 0.25) (layer "B.Cu") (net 17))
 (segment (start 107.95 101.6) (end 90.17 101.6) (width 0.25) (layer "B.Cu") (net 17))
 (segment (start 115.57 82.55) (end 117.4 80.72) (width 0.25) (layer "B.Cu") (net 17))
 (segment (start 113.03 130.81) (end 111.76 130.81) (width 0.25) (layer "B.Cu") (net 17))
 (segment (start 111.76 130.81) (end 110.49 129.54) (width 0.25) (layer "B.Cu") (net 17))
 (segment (start 92.71 82.55) (end 115.57 82.55) (width 0.25) (layer "B.Cu") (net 17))
 (segment (start 90.17 101.6) (end 90.17 85.09) (width 0.25) (layer "B.Cu") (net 17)))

